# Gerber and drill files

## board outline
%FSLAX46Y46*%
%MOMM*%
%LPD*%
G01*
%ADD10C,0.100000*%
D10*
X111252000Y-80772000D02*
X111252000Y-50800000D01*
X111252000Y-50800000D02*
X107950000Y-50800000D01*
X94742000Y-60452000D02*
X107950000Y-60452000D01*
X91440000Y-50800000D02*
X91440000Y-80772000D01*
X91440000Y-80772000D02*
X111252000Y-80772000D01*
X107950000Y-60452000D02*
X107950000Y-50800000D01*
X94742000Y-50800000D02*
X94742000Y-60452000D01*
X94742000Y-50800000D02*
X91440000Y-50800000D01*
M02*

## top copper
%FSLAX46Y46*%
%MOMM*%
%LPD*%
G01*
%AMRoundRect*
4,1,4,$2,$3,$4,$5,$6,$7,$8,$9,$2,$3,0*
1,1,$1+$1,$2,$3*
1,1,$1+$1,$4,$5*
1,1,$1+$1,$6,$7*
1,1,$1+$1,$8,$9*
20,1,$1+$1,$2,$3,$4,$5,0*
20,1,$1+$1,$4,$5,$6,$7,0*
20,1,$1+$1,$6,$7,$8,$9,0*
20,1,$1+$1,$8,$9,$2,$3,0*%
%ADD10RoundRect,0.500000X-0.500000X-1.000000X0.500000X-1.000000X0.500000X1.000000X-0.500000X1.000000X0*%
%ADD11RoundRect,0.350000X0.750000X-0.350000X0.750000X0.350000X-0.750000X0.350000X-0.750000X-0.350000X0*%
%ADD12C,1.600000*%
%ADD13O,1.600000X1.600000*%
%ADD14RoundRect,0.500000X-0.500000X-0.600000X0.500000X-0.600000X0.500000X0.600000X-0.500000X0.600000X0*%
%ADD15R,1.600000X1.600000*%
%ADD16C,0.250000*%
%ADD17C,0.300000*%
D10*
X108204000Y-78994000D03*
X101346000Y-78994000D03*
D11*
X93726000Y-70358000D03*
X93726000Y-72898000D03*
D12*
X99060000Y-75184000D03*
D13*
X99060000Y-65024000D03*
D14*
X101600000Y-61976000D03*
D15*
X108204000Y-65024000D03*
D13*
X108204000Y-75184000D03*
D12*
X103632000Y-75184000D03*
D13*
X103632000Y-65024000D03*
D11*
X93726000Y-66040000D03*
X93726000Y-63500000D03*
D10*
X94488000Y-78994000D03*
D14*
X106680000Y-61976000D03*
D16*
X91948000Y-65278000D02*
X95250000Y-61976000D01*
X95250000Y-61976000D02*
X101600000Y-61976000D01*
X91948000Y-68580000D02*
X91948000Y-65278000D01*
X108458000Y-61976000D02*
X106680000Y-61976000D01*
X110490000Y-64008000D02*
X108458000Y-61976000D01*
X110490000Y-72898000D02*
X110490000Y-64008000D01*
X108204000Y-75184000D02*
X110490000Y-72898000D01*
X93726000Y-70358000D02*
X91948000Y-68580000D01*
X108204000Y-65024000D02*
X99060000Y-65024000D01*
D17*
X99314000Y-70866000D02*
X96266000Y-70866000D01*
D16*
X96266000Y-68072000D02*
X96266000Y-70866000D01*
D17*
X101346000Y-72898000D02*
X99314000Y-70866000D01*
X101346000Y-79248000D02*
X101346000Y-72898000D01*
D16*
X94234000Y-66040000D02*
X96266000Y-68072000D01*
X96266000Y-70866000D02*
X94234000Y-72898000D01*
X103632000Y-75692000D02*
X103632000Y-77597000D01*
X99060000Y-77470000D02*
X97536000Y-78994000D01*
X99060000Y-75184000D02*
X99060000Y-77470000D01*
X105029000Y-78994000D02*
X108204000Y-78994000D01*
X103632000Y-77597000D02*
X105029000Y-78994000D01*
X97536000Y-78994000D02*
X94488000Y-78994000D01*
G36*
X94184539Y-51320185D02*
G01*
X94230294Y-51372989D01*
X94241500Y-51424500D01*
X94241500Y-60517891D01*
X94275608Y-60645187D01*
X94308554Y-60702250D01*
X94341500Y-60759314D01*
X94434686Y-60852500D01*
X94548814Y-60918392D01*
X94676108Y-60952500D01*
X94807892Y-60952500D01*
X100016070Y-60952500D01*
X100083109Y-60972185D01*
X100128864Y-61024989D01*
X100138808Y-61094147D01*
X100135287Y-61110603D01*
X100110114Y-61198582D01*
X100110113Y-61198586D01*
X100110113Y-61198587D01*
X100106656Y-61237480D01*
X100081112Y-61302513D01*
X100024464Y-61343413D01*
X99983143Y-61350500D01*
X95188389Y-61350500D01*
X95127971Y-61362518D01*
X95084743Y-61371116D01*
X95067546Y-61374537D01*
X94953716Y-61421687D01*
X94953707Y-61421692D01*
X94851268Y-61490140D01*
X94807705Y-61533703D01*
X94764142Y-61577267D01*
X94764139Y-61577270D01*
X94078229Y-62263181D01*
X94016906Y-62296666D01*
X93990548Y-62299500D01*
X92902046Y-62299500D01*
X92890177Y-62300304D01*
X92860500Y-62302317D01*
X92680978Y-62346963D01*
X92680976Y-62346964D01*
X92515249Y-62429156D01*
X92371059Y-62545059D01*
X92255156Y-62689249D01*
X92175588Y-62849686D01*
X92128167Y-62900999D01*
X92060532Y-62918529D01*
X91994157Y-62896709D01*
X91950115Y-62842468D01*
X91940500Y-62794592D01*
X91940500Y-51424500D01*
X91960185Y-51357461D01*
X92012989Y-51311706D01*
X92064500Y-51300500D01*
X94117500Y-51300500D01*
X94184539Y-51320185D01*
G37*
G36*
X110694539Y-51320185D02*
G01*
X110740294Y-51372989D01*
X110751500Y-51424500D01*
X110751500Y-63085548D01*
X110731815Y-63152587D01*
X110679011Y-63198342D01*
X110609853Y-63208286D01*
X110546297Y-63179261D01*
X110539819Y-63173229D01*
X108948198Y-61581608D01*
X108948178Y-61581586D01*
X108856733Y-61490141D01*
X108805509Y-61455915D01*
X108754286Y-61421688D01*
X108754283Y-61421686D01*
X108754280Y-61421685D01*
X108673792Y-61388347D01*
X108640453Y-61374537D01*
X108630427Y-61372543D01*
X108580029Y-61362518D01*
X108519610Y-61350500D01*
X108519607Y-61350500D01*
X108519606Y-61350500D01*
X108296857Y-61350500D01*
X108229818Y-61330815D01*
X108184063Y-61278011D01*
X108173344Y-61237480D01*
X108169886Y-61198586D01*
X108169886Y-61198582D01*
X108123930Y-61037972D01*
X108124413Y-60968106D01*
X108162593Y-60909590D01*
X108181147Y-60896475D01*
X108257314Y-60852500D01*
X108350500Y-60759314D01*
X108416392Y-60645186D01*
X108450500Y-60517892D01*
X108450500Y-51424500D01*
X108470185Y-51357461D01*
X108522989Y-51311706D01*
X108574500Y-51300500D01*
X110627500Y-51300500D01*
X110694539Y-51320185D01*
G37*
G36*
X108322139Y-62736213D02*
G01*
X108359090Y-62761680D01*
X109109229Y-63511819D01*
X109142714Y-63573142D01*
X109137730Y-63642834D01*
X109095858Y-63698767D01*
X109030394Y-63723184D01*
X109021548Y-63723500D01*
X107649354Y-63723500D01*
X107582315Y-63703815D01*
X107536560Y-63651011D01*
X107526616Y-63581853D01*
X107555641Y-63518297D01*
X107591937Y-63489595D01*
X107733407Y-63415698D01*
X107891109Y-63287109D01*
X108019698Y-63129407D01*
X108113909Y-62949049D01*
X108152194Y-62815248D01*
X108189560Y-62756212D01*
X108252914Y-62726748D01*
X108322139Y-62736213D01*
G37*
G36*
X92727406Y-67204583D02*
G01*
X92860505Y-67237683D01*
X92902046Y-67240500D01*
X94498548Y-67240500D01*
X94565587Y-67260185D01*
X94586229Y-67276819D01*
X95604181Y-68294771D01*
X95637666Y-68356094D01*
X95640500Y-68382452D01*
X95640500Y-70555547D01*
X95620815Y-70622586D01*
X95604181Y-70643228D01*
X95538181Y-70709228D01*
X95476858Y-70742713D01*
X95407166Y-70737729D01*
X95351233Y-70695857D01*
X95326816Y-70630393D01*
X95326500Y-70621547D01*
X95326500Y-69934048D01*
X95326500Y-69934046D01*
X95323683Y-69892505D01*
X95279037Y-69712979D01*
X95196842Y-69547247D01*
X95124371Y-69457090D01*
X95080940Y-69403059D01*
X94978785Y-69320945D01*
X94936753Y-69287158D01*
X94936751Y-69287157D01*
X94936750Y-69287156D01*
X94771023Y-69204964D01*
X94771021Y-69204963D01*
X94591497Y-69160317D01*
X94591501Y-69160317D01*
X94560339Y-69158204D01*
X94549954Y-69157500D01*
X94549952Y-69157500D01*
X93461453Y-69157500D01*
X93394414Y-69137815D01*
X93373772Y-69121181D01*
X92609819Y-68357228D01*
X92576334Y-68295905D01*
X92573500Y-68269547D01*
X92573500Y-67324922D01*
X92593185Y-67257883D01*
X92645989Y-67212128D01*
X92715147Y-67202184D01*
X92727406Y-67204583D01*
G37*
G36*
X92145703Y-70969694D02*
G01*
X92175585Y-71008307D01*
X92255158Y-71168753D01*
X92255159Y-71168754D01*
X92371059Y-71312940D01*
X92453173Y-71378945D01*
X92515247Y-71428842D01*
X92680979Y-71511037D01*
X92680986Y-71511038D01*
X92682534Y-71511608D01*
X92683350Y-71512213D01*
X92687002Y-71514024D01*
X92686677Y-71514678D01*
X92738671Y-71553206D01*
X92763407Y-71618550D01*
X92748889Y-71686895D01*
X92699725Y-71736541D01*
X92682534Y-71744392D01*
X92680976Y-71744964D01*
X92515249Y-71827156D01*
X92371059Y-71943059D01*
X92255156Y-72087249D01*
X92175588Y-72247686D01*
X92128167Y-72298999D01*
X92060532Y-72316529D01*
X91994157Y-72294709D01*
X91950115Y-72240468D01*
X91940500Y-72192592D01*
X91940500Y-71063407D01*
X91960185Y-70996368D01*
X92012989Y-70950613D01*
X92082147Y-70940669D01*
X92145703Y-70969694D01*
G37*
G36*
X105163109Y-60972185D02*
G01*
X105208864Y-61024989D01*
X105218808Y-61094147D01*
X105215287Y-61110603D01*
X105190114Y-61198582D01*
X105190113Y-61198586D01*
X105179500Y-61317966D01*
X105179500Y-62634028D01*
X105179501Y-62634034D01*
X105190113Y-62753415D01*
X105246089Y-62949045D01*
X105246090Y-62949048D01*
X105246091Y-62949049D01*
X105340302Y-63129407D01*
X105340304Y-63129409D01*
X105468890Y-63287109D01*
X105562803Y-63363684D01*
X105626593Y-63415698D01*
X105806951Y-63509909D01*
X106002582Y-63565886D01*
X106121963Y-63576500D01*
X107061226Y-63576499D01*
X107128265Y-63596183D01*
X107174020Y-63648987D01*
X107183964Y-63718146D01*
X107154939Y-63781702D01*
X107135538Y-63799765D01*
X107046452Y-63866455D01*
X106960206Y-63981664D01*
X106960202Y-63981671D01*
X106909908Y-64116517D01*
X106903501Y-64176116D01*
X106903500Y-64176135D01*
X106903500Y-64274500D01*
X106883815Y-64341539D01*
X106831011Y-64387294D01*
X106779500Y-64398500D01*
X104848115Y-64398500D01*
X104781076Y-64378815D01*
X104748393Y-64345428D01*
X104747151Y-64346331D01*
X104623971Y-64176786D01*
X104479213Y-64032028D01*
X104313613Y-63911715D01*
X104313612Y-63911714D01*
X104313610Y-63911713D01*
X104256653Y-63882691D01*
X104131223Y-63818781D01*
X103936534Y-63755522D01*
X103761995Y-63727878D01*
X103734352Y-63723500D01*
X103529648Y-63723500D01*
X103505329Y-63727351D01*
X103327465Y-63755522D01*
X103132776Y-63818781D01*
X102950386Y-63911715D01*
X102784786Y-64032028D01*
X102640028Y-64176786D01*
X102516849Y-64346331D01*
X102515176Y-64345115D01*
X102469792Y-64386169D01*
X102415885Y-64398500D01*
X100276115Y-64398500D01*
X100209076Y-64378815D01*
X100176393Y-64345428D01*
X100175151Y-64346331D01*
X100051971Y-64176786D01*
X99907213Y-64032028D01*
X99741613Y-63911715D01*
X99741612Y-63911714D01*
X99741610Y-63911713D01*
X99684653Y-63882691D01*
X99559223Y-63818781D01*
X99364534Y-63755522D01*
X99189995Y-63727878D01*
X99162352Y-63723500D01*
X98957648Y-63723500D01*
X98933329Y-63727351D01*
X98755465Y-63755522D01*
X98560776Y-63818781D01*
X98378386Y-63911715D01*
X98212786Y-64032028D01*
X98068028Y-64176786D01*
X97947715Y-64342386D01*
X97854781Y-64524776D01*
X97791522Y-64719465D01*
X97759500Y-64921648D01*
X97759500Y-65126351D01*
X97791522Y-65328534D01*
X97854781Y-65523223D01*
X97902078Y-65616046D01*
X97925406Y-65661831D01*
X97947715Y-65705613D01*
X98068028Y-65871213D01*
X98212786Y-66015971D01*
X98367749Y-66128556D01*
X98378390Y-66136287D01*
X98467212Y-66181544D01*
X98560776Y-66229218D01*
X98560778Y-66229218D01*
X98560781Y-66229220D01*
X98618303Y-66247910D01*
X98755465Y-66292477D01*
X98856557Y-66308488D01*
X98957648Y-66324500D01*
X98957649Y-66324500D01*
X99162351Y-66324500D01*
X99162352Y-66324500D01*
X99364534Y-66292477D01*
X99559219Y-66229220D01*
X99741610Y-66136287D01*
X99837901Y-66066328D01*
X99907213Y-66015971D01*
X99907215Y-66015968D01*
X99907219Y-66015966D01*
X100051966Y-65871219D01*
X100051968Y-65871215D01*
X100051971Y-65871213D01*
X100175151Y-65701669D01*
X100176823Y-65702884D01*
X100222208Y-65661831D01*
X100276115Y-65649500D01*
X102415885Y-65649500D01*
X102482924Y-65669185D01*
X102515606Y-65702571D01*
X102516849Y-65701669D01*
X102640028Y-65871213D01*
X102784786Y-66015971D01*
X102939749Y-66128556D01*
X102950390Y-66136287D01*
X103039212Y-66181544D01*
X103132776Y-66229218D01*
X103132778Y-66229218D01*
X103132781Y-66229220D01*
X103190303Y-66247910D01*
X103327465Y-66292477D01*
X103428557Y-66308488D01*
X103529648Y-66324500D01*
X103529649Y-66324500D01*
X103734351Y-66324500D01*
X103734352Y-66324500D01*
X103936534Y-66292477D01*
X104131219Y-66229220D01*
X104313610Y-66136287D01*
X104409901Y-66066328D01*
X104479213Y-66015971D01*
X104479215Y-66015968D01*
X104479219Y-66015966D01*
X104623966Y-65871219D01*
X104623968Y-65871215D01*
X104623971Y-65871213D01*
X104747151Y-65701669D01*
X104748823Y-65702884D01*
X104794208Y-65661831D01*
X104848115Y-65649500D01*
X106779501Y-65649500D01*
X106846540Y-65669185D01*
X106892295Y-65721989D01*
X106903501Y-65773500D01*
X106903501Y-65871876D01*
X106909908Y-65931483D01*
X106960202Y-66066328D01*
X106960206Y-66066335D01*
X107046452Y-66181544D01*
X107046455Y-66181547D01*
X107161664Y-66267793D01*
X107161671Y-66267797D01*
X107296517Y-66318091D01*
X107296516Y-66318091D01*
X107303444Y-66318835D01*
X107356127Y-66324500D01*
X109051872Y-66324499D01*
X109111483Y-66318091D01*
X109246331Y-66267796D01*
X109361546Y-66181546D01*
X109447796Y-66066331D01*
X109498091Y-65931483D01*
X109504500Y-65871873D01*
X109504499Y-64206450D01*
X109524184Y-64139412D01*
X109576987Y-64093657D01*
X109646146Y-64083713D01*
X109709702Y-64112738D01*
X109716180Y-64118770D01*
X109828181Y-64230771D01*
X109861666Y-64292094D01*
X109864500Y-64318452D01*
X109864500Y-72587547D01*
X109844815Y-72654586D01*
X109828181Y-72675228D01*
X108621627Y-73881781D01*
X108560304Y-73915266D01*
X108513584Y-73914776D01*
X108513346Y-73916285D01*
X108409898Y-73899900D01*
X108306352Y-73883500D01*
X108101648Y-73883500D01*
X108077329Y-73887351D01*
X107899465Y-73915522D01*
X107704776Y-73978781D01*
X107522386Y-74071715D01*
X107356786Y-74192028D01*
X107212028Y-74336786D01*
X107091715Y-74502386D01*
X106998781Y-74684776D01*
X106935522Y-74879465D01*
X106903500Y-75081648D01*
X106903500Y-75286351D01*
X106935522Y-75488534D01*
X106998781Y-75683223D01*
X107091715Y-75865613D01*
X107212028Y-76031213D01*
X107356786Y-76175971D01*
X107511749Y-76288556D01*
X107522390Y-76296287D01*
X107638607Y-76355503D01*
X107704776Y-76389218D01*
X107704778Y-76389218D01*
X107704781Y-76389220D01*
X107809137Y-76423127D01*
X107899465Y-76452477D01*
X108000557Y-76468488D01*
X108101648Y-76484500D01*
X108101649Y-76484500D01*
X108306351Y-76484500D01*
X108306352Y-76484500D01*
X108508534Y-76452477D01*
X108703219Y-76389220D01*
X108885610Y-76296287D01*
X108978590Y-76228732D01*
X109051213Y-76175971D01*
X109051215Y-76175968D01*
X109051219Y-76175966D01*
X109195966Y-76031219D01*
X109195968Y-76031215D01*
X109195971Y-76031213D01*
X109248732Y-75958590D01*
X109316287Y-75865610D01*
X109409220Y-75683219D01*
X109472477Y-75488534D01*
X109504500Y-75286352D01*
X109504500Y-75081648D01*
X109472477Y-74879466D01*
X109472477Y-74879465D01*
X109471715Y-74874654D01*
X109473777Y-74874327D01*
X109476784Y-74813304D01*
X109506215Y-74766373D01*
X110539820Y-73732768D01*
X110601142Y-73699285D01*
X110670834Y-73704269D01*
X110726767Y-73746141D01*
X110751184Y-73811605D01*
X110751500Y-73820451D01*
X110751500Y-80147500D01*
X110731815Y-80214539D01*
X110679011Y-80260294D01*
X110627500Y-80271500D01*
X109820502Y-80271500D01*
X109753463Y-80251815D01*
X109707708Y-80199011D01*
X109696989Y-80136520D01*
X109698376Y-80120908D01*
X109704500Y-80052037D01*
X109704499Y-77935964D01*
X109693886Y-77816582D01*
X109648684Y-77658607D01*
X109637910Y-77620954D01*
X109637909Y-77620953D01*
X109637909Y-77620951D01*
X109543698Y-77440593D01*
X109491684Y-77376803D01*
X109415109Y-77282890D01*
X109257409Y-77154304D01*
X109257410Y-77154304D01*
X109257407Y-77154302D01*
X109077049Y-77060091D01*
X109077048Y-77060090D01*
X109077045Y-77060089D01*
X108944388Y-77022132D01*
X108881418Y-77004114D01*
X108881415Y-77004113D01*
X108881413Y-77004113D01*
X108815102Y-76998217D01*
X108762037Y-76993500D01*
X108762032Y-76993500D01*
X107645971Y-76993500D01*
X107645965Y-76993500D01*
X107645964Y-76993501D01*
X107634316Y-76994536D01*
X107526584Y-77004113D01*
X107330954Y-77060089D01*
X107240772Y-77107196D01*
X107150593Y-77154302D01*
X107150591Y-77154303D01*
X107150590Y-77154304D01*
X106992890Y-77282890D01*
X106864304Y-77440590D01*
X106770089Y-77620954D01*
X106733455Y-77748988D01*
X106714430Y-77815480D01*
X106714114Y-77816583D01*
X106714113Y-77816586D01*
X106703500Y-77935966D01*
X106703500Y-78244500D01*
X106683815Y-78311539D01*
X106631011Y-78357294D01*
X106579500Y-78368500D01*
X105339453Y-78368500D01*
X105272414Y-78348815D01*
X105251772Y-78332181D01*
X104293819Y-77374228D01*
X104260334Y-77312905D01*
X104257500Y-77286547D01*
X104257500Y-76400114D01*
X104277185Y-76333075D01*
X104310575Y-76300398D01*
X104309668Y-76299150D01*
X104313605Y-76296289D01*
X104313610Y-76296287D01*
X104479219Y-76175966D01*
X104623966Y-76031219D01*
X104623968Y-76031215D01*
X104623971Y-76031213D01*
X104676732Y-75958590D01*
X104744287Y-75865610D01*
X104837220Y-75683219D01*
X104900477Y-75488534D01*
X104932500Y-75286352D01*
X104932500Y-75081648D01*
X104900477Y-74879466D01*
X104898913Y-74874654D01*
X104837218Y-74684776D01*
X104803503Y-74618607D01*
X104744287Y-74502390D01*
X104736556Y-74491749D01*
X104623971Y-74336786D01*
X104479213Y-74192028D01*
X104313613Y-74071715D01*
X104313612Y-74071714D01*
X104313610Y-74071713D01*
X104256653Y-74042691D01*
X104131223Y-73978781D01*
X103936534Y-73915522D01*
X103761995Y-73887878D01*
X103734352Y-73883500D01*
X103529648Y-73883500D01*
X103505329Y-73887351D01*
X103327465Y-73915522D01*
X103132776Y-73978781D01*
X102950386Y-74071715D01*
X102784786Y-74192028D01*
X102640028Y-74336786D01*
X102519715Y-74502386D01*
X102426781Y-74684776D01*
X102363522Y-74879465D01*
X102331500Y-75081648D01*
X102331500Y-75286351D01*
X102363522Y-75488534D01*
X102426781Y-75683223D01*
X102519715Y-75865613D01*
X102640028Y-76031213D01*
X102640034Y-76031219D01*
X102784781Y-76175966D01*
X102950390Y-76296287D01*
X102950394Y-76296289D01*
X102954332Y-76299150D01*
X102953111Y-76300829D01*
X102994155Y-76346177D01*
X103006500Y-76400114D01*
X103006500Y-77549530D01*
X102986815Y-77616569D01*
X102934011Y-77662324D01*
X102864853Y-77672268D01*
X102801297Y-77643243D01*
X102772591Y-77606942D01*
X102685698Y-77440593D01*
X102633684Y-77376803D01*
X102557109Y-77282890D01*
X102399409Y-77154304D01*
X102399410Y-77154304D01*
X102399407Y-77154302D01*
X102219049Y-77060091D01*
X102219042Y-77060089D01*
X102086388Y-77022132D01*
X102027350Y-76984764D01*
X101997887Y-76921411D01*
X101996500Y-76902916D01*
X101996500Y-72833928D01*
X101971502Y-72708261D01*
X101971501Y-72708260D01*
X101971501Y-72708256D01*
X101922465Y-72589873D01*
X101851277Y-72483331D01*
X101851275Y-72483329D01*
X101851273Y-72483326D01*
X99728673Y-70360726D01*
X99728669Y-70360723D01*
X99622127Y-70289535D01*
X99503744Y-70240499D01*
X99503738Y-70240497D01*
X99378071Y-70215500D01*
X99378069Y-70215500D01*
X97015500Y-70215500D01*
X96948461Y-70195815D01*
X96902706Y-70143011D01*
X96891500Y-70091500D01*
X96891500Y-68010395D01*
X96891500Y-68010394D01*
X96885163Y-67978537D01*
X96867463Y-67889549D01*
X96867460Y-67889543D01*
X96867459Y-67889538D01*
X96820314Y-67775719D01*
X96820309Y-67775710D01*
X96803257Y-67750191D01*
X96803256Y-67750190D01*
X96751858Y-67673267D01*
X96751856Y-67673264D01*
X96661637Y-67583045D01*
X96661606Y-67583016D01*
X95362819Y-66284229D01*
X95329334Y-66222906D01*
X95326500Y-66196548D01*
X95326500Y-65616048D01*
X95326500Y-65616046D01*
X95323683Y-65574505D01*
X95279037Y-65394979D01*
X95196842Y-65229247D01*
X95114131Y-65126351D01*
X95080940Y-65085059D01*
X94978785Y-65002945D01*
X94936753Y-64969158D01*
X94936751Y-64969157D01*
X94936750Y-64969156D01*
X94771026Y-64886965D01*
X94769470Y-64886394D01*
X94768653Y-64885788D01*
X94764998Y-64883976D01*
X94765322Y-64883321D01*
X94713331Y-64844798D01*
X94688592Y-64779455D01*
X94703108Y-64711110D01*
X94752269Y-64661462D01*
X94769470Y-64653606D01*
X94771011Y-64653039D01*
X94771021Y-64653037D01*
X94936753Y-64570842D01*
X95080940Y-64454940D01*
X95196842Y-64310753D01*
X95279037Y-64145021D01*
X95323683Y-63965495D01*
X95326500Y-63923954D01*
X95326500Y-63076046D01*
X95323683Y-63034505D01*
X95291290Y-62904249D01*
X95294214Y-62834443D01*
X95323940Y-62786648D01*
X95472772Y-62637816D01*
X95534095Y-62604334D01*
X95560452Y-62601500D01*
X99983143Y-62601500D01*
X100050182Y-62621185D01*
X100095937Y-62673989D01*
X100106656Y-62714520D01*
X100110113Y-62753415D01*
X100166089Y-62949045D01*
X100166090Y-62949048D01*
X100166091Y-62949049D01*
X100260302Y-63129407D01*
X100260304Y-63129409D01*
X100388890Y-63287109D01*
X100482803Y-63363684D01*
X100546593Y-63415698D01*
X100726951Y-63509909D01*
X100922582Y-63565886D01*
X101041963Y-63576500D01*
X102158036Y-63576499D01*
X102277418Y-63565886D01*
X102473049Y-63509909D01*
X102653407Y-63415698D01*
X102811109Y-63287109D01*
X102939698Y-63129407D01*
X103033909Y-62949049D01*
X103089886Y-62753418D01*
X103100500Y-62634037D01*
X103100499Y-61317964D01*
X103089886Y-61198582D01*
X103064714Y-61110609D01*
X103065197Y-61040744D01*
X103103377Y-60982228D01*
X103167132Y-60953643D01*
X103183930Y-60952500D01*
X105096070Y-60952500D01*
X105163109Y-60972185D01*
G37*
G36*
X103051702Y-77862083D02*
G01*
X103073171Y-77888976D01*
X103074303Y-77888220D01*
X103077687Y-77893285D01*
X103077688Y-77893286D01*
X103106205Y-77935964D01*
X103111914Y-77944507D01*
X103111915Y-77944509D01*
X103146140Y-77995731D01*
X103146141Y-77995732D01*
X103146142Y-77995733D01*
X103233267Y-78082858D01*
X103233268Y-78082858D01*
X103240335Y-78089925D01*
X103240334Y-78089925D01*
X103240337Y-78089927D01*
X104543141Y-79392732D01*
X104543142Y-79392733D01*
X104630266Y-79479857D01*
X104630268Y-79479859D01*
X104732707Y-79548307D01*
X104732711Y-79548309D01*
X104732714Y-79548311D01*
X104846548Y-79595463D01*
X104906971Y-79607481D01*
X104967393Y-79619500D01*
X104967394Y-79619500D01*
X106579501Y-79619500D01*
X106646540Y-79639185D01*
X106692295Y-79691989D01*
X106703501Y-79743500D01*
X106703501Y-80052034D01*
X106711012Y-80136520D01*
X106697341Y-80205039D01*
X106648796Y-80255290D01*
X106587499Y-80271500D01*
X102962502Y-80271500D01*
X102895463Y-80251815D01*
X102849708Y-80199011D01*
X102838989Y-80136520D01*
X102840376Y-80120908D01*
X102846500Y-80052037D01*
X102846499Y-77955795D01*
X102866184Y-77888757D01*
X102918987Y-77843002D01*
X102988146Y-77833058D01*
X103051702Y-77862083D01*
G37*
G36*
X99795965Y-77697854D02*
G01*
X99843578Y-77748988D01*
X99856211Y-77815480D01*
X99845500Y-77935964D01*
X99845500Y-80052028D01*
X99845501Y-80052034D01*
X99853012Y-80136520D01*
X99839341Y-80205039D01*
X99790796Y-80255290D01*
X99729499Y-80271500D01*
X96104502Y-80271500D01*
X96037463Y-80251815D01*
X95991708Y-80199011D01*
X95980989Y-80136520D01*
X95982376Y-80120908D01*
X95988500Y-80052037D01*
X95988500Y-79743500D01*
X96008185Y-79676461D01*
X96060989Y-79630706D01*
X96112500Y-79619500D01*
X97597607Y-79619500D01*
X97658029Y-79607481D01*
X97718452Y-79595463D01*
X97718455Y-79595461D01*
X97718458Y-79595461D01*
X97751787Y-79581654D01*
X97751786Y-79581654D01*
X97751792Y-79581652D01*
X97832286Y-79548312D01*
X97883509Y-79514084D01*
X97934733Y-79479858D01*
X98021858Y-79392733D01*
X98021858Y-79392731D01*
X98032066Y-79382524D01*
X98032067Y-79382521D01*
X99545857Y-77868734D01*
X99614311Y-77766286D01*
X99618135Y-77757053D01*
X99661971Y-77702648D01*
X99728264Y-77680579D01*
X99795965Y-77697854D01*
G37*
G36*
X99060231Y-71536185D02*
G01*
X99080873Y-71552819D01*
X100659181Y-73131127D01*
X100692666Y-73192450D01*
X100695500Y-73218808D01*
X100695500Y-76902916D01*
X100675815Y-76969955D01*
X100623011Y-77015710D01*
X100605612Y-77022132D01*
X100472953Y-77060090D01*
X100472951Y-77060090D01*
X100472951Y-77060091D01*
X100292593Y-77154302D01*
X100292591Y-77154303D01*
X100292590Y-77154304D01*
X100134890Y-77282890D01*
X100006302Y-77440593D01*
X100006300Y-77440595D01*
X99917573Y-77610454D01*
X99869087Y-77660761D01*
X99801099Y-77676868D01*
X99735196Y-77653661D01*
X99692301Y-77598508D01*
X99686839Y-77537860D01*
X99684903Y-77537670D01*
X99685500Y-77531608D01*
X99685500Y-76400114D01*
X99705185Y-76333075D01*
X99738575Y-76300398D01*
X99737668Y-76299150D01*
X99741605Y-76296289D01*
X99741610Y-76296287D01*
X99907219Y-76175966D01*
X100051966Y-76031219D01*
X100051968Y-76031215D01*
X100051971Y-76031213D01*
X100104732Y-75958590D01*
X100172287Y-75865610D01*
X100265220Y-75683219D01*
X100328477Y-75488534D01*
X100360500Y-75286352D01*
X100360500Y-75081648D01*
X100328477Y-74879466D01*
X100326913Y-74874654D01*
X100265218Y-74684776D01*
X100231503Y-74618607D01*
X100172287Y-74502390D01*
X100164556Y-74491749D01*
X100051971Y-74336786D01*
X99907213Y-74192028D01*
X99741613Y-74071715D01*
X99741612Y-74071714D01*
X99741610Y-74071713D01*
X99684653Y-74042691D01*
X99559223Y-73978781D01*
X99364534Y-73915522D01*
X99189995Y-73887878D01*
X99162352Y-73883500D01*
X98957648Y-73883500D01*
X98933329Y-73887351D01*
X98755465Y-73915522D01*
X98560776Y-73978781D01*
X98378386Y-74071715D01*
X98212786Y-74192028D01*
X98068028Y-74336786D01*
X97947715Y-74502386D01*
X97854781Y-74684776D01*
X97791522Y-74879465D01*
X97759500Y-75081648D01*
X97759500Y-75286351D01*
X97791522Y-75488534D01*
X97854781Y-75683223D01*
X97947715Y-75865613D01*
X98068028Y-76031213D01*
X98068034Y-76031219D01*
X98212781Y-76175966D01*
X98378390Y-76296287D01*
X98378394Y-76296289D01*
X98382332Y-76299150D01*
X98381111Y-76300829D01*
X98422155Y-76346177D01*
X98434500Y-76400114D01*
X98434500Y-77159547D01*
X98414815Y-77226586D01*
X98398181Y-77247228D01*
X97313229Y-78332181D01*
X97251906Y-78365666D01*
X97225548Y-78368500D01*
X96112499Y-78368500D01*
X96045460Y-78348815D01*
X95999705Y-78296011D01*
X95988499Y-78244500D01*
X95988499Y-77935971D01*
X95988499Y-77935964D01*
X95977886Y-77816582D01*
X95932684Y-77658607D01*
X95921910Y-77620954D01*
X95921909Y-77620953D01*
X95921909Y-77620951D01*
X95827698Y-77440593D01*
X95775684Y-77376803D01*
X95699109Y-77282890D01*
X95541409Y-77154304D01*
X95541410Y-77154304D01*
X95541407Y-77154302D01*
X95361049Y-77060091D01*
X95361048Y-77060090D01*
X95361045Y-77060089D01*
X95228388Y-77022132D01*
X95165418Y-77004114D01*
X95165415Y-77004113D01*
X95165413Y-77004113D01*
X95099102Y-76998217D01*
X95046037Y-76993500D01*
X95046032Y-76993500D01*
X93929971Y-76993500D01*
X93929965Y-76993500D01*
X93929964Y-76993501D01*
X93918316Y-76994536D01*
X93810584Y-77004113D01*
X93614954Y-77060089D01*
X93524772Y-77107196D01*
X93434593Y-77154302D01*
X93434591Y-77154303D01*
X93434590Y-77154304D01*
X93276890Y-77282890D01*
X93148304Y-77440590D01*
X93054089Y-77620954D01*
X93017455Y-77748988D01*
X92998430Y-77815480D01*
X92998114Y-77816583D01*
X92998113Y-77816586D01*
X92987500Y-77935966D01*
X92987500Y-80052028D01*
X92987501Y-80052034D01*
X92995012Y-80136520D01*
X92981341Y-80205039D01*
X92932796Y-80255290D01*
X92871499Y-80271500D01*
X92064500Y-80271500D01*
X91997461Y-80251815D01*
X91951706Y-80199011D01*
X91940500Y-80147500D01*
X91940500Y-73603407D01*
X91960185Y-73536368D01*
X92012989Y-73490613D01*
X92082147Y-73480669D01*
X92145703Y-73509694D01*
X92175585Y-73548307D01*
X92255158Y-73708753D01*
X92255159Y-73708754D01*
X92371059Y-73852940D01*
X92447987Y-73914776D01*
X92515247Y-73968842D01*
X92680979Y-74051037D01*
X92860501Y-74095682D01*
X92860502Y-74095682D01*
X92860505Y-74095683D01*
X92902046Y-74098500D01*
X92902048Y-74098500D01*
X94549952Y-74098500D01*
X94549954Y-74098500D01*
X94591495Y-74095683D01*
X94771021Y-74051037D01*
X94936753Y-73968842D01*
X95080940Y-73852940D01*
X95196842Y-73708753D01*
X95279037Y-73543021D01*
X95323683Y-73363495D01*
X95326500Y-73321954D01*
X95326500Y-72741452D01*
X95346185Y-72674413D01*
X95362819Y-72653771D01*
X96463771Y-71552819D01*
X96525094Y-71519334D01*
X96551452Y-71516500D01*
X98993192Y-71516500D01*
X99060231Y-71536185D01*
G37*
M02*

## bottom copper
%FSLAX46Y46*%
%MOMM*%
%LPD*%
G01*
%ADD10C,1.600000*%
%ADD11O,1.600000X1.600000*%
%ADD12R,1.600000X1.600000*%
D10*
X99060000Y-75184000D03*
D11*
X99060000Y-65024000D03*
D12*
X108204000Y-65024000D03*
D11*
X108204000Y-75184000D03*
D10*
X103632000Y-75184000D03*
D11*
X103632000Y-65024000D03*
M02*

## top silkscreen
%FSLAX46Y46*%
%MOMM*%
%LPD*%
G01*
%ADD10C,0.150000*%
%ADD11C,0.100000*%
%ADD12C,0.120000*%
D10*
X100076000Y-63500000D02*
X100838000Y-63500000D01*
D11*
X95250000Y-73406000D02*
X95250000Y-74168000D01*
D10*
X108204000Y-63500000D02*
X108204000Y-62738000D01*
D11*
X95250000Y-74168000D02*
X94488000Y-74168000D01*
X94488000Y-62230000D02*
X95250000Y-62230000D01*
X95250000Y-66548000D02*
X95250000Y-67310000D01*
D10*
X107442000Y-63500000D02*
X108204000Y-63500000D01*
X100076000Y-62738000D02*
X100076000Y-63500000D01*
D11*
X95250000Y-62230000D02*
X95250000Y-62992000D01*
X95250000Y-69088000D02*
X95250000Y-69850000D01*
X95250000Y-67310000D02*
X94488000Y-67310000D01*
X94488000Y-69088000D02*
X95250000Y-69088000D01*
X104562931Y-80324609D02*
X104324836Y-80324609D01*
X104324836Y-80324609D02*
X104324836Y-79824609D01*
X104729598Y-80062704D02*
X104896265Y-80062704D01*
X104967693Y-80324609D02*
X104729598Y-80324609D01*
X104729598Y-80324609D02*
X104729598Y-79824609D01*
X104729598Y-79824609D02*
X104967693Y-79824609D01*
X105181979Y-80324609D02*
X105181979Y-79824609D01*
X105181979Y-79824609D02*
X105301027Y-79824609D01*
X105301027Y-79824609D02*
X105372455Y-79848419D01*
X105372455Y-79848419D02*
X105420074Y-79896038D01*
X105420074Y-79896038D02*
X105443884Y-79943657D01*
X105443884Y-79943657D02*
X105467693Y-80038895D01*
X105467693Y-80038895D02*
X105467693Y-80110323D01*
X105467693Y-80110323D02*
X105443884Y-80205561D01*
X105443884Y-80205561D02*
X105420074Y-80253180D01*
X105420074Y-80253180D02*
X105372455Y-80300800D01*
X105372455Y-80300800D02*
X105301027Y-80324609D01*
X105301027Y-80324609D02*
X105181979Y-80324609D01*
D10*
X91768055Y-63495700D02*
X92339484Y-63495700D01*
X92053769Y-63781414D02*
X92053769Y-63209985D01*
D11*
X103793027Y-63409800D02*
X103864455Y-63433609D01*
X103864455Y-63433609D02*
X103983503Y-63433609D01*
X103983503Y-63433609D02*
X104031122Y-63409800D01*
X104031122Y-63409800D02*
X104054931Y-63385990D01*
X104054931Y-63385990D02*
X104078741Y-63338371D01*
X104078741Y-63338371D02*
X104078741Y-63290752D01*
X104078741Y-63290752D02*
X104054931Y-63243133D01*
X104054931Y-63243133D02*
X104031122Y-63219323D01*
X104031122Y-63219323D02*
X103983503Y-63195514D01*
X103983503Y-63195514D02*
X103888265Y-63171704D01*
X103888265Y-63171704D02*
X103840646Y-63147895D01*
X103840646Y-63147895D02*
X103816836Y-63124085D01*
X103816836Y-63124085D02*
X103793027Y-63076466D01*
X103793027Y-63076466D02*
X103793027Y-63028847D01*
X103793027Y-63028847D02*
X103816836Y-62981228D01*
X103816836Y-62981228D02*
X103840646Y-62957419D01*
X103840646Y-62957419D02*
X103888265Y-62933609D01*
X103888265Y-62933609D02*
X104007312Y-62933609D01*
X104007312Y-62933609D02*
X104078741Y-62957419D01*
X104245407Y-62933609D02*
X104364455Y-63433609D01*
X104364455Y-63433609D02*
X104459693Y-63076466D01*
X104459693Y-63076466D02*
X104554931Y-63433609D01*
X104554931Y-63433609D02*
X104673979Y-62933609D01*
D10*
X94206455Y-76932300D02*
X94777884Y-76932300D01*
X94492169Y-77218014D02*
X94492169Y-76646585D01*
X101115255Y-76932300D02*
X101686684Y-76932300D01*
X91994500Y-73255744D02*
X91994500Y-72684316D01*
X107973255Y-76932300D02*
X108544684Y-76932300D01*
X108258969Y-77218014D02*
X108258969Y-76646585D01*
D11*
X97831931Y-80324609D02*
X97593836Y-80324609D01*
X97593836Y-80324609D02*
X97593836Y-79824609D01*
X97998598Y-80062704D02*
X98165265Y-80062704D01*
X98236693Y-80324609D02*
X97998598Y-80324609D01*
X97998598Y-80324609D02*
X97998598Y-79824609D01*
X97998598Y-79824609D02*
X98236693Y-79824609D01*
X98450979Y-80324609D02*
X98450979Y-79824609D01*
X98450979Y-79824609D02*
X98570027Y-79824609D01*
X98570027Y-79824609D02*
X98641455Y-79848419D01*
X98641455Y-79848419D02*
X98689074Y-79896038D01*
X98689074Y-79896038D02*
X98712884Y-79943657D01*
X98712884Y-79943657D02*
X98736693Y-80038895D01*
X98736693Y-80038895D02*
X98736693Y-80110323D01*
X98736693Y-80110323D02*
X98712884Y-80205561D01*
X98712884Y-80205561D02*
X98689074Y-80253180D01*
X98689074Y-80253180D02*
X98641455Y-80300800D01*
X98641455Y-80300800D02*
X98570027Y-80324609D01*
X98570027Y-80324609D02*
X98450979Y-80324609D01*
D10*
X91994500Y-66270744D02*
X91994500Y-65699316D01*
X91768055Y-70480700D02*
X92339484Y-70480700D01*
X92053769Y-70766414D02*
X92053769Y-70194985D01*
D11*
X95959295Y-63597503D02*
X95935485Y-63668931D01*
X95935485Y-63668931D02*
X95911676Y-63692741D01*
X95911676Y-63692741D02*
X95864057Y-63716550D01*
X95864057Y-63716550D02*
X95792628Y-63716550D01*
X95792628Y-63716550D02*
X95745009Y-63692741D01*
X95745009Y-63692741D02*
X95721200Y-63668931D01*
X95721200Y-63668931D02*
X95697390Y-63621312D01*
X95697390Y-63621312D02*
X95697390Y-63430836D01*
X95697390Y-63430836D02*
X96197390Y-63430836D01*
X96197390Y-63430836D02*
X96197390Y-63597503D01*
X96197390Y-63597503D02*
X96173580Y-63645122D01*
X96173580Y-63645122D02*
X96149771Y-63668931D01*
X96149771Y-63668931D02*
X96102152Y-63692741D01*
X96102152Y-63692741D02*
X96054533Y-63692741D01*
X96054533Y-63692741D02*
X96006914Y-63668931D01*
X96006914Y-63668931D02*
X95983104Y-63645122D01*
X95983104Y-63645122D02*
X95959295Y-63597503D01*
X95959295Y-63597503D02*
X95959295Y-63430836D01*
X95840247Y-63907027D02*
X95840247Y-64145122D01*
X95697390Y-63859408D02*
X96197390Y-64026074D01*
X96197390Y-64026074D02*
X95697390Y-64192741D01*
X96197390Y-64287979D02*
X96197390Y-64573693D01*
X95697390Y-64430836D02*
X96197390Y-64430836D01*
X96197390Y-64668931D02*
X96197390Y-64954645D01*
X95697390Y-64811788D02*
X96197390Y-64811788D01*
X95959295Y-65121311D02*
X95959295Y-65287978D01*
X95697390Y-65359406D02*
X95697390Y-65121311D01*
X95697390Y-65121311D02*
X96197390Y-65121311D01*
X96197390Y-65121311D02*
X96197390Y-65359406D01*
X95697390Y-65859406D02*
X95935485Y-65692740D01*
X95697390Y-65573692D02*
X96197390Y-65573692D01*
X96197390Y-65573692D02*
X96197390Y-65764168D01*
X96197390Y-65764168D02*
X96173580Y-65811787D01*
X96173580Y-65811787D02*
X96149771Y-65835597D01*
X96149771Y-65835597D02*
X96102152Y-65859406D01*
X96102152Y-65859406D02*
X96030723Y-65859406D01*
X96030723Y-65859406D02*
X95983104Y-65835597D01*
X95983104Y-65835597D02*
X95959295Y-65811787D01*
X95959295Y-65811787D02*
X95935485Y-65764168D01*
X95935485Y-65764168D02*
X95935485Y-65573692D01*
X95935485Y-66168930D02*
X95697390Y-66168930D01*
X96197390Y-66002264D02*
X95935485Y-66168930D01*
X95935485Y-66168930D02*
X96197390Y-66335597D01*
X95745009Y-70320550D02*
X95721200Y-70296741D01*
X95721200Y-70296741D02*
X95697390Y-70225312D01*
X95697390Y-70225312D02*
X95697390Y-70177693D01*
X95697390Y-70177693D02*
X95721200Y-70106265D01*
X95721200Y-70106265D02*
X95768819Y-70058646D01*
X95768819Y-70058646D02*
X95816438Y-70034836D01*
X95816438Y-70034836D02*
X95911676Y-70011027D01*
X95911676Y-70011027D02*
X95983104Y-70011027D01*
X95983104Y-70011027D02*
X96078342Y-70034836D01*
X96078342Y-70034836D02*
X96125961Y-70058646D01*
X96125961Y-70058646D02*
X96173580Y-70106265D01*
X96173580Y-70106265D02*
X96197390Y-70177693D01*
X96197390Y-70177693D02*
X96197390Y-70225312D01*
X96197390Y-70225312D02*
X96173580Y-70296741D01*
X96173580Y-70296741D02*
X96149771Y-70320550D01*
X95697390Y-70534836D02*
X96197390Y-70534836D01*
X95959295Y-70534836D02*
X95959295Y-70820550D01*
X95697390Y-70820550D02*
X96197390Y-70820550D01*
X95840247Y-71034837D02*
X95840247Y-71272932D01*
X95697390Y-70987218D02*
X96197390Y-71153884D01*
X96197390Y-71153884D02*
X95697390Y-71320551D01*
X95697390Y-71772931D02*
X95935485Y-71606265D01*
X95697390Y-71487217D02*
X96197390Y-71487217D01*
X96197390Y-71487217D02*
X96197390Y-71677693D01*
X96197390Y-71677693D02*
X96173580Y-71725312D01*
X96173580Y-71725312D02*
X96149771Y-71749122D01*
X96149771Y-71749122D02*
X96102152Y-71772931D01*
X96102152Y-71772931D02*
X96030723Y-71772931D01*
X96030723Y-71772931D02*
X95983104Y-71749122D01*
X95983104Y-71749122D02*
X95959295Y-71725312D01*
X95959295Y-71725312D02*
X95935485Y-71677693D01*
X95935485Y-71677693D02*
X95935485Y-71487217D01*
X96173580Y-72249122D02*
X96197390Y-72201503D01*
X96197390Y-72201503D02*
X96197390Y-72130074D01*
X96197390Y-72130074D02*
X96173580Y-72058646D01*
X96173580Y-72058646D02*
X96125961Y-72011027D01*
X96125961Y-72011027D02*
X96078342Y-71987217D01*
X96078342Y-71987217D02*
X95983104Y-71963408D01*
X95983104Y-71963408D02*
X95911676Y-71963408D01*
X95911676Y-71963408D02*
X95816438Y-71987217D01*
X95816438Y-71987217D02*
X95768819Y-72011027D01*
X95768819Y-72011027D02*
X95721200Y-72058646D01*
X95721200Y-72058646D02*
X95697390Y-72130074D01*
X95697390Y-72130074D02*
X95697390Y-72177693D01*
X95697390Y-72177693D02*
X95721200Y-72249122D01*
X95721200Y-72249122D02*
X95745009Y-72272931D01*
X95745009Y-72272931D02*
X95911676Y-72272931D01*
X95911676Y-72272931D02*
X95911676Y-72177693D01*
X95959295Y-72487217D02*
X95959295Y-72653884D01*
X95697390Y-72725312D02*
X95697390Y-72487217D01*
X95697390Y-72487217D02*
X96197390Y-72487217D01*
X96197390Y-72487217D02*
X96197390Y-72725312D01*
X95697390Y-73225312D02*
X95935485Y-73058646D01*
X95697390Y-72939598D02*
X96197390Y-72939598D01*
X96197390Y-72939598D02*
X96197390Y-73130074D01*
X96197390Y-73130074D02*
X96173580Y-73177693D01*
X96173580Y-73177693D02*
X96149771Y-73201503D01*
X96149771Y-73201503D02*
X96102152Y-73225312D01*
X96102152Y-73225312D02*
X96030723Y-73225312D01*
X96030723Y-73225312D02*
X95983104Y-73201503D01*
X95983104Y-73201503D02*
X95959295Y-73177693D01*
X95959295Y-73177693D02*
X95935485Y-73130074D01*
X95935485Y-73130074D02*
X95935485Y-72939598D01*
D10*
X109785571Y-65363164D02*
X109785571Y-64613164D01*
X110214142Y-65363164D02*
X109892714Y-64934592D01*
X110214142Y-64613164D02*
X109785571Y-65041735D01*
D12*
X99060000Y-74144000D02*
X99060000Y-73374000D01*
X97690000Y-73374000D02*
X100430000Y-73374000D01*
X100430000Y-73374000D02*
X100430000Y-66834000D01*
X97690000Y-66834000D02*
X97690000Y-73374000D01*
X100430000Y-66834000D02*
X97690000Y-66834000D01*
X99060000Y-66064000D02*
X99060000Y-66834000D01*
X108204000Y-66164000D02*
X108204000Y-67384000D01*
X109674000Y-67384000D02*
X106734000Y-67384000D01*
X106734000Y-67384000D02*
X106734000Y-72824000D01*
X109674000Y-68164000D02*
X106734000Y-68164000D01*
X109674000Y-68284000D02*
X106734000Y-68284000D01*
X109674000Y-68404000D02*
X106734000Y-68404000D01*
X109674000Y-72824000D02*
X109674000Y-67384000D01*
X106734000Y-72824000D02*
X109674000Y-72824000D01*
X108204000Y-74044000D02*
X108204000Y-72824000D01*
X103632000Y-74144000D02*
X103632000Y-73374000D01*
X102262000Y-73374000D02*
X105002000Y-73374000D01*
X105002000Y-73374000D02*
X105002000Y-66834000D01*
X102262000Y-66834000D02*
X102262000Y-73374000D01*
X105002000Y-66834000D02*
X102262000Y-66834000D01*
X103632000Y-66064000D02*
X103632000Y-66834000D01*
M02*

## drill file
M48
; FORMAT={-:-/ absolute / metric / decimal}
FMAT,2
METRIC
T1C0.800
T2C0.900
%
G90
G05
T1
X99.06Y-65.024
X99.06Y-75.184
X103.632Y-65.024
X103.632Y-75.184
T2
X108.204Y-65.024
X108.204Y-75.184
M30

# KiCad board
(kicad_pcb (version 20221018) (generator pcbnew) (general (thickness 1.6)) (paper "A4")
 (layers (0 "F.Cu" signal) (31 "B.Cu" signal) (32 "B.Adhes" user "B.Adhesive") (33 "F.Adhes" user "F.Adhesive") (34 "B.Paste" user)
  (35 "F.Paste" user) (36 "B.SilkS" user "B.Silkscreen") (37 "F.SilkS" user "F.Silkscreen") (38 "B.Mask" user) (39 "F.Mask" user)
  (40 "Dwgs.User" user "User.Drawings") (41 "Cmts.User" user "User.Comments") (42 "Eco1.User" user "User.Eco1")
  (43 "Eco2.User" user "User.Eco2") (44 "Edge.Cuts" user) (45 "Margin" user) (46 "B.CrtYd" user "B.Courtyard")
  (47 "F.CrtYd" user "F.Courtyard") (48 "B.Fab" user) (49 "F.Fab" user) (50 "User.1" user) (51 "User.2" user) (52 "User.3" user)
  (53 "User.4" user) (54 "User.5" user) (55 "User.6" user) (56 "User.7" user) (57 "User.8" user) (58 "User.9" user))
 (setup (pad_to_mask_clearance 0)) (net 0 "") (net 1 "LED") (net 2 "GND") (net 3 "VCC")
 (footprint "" (layer "F.Cu") (at 108.204 78.994)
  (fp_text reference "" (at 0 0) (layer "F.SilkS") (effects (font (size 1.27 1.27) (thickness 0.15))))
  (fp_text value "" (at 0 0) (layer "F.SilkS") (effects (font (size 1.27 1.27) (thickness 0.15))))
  (pad "" connect roundrect (at 0 0) (size 2 3) (layers "F.Cu" "F.Mask") (roundrect_rratio 0.25) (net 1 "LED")))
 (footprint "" (layer "F.Cu") (at 101.346 78.994)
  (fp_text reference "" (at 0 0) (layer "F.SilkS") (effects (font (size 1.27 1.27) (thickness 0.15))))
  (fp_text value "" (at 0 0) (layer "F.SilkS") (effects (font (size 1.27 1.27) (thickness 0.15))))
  (pad "" connect roundrect (at 0 0) (size 2 3) (layers "F.Cu" "F.Mask") (roundrect_rratio 0.25) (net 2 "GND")))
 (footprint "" (layer "F.Cu") (at 93.726 70.358 90)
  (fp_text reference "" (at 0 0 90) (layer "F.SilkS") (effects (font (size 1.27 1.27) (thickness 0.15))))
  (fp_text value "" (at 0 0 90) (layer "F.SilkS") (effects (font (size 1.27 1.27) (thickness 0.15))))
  (pad "" connect roundrect (at 0 0 90) (size 1.4 2.2) (layers "F.Cu" "F.Mask") (roundrect_rratio 0.25) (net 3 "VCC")))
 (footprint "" (layer "F.Cu") (at 93.726 72.898 90)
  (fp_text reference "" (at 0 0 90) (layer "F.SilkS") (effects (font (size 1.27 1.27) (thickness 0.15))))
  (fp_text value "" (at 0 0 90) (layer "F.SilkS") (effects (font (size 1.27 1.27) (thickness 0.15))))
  (pad "" connect roundrect (at 0 0 90) (size 1.4 2.2) (layers "F.Cu" "F.Mask") (roundrect_rratio 0.25) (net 2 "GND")))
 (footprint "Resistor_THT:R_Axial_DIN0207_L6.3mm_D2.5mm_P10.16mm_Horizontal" (layer "F.Cu") (at 99.06 75.184 90)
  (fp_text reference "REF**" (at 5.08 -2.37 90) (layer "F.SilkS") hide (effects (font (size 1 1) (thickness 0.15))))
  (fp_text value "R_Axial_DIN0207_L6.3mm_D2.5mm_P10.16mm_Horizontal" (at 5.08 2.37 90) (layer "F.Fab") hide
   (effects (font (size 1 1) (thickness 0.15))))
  (fp_line (start 1.04 0) (end 1.81 0) (stroke (width 0.12) (type solid)) (layer "F.SilkS"))
  (fp_line (start 1.81 -1.37) (end 1.81 1.37) (stroke (width 0.12) (type solid)) (layer "F.SilkS"))
  (fp_line (start 1.81 1.37) (end 8.35 1.37) (stroke (width 0.12) (type solid)) (layer "F.SilkS"))
  (fp_line (start 8.35 -1.37) (end 1.81 -1.37) (stroke (width 0.12) (type solid)) (layer "F.SilkS"))
  (fp_line (start 8.35 1.37) (end 8.35 -1.37) (stroke (width 0.12) (type solid)) (layer "F.SilkS"))
  (fp_line (start 9.12 0) (end 8.35 0) (stroke (width 0.12) (type solid)) (layer "F.SilkS"))
  (pad "1" thru_hole circle (at 0 0 90) (size 1.6 1.6) (drill 0.8) (layers "*.Cu" "*.Mask") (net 1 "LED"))
  (pad "2" thru_hole oval (at 10.16 0 90) (size 1.6 1.6) (drill 0.8) (layers "*.Cu" "*.Mask") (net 3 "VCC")))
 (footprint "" (layer "F.Cu") (at 101.6 61.976)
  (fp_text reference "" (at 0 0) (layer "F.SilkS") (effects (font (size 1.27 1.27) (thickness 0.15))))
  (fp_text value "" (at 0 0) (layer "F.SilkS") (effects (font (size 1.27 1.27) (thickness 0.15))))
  (pad "" connect roundrect (at 0 0) (size 2 2.2) (layers "F.Cu" "F.Mask") (roundrect_rratio 0.25) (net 3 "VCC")))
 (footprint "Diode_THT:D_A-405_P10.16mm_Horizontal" (layer "F.Cu") (at 108.204 65.024 -90)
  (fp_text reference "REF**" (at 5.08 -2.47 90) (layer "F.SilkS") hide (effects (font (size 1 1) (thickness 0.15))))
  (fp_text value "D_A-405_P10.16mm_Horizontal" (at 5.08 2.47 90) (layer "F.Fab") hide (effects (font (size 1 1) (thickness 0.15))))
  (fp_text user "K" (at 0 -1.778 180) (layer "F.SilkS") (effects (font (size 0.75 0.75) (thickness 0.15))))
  (fp_line (start 1.14 0) (end 2.36 0) (stroke (width 0.12) (type solid)) (layer "F.SilkS"))
  (fp_line (start 2.36 -1.47) (end 2.36 1.47) (stroke (width 0.12) (type solid)) (layer "F.SilkS"))
  (fp_line (start 2.36 1.47) (end 7.8 1.47) (stroke (width 0.12) (type solid)) (layer "F.SilkS"))
  (fp_line (start 3.14 -1.47) (end 3.14 1.47) (stroke (width 0.12) (type solid)) (layer "F.SilkS"))
  (fp_line (start 3.26 -1.47) (end 3.26 1.47) (stroke (width 0.12) (type solid)) (layer "F.SilkS"))
  (fp_line (start 3.38 -1.47) (end 3.38 1.47) (stroke (width 0.12) (type solid)) (layer "F.SilkS"))
  (fp_line (start 7.8 -1.47) (end 2.36 -1.47) (stroke (width 0.12) (type solid)) (layer "F.SilkS"))
  (fp_line (start 7.8 1.47) (end 7.8 -1.47) (stroke (width 0.12) (type solid)) (layer "F.SilkS"))
  (fp_line (start 9.02 0) (end 7.8 0) (stroke (width 0.12) (type solid)) (layer "F.SilkS"))
  (pad "1" thru_hole rect (at 0 0 270) (size 1.6 1.6) (drill 0.9) (layers "*.Cu" "*.Mask") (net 3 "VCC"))
  (pad "2" thru_hole oval (at 10.16 0 270) (size 1.6 1.6) (drill 0.9) (layers "*.Cu" "*.Mask") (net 3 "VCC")))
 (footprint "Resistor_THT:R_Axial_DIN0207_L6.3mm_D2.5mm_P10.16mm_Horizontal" (layer "F.Cu") (at 103.632 75.184 90)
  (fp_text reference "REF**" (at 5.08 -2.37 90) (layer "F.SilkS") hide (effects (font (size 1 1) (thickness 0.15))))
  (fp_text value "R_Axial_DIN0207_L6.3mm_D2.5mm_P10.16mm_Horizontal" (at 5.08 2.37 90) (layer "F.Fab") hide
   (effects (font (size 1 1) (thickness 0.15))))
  (fp_line (start 1.04 0) (end 1.81 0) (stroke (width 0.12) (type solid)) (layer "F.SilkS"))
  (fp_line (start 1.81 -1.37) (end 1.81 1.37) (stroke (width 0.12) (type solid)) (layer "F.SilkS"))
  (fp_line (start 1.81 1.37) (end 8.35 1.37) (stroke (width 0.12) (type solid)) (layer "F.SilkS"))
  (fp_line (start 8.35 -1.37) (end 1.81 -1.37) (stroke (width 0.12) (type solid)) (layer "F.SilkS"))
  (fp_line (start 8.35 1.37) (end 8.35 -1.37) (stroke (width 0.12) (type solid)) (layer "F.SilkS"))
  (fp_line (start 9.12 0) (end 8.35 0) (stroke (width 0.12) (type solid)) (layer "F.SilkS"))
  (pad "1" thru_hole circle (at 0 0 90) (size 1.6 1.6) (drill 0.8) (layers "*.Cu" "*.Mask") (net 1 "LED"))
  (pad "2" thru_hole oval (at 10.16 0 90) (size 1.6 1.6) (drill 0.8) (layers "*.Cu" "*.Mask") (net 3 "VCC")))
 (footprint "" (layer "F.Cu") (at 93.726 66.04 90)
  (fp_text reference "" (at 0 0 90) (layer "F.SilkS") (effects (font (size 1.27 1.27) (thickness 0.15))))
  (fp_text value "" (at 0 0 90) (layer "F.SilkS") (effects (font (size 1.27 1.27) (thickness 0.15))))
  (pad "" connect roundrect (at 0 0 90) (size 1.4 2.2) (layers "F.Cu" "F.Mask") (roundrect_rratio 0.25) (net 2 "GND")))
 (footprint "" (layer "F.Cu") (at 93.726 63.5 90)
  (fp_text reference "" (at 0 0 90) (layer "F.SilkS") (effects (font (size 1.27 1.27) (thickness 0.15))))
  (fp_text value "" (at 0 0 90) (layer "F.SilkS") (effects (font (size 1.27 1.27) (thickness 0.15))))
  (pad "" connect roundrect (at 0 0 90) (size 1.4 2.2) (layers "F.Cu" "F.Mask") (roundrect_rratio 0.25) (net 3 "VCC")))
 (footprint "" (layer "F.Cu") (at 94.488 78.994)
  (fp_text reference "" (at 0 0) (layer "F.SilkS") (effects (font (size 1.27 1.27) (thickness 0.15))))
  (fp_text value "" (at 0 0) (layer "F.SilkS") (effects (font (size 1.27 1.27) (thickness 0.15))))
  (pad "" connect roundrect (at 0 0) (size 2 3) (layers "F.Cu" "F.Mask") (roundrect_rratio 0.25) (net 1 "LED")))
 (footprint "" (layer "F.Cu") (at 106.68 61.976)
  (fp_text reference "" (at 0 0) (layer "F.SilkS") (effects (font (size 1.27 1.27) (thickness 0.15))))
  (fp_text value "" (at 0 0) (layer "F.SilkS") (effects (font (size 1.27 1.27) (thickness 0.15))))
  (pad "" connect roundrect (at 0 0) (size 2 2.2) (layers "F.Cu" "F.Mask") (roundrect_rratio 0.25) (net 3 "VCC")))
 (gr_line (start 100.076 63.5) (end 100.838 63.5) (stroke (width 0.15) (type default)) (layer "F.SilkS"))
 (gr_line (start 95.25 73.406) (end 95.25 74.168) (stroke (width 0.1) (type default)) (layer "F.SilkS"))
 (gr_line (start 108.204 63.5) (end 108.204 62.738) (stroke (width 0.15) (type default)) (layer "F.SilkS"))
 (gr_line (start 95.25 74.168) (end 94.488 74.168) (stroke (width 0.1) (type default)) (layer "F.SilkS"))
 (gr_line (start 94.488 62.23) (end 95.25 62.23) (stroke (width 0.1) (type default)) (layer "F.SilkS"))
 (gr_line (start 95.25 66.548) (end 95.25 67.31) (stroke (width 0.1) (type default)) (layer "F.SilkS"))
 (gr_line (start 107.442 63.5) (end 108.204 63.5) (stroke (width 0.15) (type default)) (layer "F.SilkS"))
 (gr_line (start 100.076 62.738) (end 100.076 63.5) (stroke (width 0.15) (type default)) (layer "F.SilkS"))
 (gr_line (start 95.25 62.23) (end 95.25 62.992) (stroke (width 0.1) (type default)) (layer "F.SilkS"))
 (gr_line (start 95.25 69.088) (end 95.25 69.85) (stroke (width 0.1) (type default)) (layer "F.SilkS"))
 (gr_line (start 95.25 67.31) (end 94.488 67.31) (stroke (width 0.1) (type default)) (layer "F.SilkS"))
 (gr_line (start 94.488 69.088) (end 95.25 69.088) (stroke (width 0.1) (type default)) (layer "F.SilkS"))
 (gr_line (start 111.252 80.772) (end 111.252 50.8) (stroke (width 0.1) (type default)) (layer "Edge.Cuts"))
 (gr_line (start 111.252 50.8) (end 107.95 50.8) (stroke (width 0.1) (type default)) (layer "Edge.Cuts"))
 (gr_line (start 94.742 60.452) (end 107.95 60.452) (stroke (width 0.1) (type default)) (layer "Edge.Cuts"))
 (gr_line (start 91.44 50.8) (end 91.44 80.772) (stroke (width 0.1) (type default)) (layer "Edge.Cuts"))
 (gr_line (start 91.44 80.772) (end 111.252 80.772) (stroke (width 0.1) (type default)) (layer "Edge.Cuts"))
 (gr_line (start 107.95 60.452) (end 107.95 50.8) (stroke (width 0.1) (type default)) (layer "Edge.Cuts"))
 (gr_line (start 94.742 50.8) (end 94.742 60.452) (stroke (width 0.1) (type default)) (layer "Edge.Cuts"))
 (gr_line (start 94.742 50.8) (end 91.44 50.8) (stroke (width 0.1) (type default)) (layer "Edge.Cuts"))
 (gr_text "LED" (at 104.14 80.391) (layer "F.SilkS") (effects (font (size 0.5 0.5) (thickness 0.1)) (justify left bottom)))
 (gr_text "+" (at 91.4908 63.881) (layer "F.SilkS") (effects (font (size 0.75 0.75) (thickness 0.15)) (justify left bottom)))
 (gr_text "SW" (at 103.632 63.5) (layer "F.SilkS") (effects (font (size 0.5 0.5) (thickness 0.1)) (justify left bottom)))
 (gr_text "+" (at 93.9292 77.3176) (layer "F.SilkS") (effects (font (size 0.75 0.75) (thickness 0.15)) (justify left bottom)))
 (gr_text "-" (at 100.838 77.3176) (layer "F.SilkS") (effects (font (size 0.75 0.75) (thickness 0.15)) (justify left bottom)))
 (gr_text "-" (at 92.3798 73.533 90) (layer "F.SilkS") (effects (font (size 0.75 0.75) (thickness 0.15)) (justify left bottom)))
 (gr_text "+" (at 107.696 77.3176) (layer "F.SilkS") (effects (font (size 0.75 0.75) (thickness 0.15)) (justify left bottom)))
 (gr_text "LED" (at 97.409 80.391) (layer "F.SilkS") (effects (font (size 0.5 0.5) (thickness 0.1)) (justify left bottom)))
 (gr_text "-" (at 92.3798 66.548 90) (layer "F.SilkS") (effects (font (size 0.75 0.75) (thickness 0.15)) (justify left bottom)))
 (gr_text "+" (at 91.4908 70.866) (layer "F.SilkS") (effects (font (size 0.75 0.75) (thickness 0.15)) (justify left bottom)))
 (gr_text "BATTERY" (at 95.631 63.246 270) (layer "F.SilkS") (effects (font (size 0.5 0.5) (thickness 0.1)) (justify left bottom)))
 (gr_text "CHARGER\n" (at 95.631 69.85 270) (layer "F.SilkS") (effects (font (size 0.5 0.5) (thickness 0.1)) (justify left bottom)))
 (segment (start 91.948 65.278) (end 95.25 61.976) (width 0.25) (layer "F.Cu") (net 3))
 (segment (start 95.25 61.976) (end 101.6 61.976) (width 0.25) (layer "F.Cu") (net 3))
 (segment (start 91.948 68.58) (end 91.948 65.278) (width 0.25) (layer "F.Cu") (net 3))
 (segment (start 108.458 61.976) (end 106.68 61.976) (width 0.25) (layer "F.Cu") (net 3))
 (segment (start 110.49 64.008) (end 108.458 61.976) (width 0.25) (layer "F.Cu") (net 3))
 (segment (start 110.49 72.898) (end 110.49 64.008) (width 0.25) (layer "F.Cu") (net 3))
 (segment (start 108.204 75.184) (end 110.49 72.898) (width 0.25) (layer "F.Cu") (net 3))
 (segment (start 93.726 70.358) (end 91.948 68.58) (width 0.25) (layer "F.Cu") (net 3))
 (segment (start 108.204 65.024) (end 99.06 65.024) (width 0.25) (layer "F.Cu") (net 3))
 (segment (start 99.314 70.866) (end 96.266 70.866) (width 0.3) (layer "F.Cu") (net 2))
 (segment (start 96.266 68.072) (end 96.266 70.866) (width 0.25) (layer "F.Cu") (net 2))
 (segment (start 101.346 72.898) (end 99.314 70.866) (width 0.3) (layer "F.Cu") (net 2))
 (segment (start 101.346 79.248) (end 101.346 72.898) (width 0.3) (layer "F.Cu") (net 2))
 (segment (start 94.234 66.04) (end 96.266 68.072) (width 0.25) (layer "F.Cu") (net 2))
 (segment (start 96.266 70.866) (end 94.234 72.898) (width 0.25) (layer "F.Cu") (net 2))
 (segment (start 103.632 75.692) (end 103.632 77.597) (width 0.25) (layer "F.Cu") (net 1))
 (segment (start 99.06 77.47) (end 97.536 78.994) (width 0.25) (layer "F.Cu") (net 1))
 (segment (start 99.06 75.184) (end 99.06 77.47) (width 0.25) (layer "F.Cu") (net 1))
 (segment (start 105.029 78.994) (end 108.204 78.994) (width 0.25) (layer "F.Cu") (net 1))
 (segment (start 103.632 77.597) (end 105.029 78.994) (width 0.25) (layer "F.Cu") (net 1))
 (segment (start 97.536 78.994) (end 94.488 78.994) (width 0.25) (layer "F.Cu") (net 1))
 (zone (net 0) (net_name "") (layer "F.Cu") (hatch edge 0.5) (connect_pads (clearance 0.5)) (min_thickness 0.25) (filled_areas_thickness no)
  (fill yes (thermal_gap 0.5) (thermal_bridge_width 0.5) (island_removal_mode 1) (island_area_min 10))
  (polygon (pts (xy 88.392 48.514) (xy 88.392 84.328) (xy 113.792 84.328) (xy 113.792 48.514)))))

